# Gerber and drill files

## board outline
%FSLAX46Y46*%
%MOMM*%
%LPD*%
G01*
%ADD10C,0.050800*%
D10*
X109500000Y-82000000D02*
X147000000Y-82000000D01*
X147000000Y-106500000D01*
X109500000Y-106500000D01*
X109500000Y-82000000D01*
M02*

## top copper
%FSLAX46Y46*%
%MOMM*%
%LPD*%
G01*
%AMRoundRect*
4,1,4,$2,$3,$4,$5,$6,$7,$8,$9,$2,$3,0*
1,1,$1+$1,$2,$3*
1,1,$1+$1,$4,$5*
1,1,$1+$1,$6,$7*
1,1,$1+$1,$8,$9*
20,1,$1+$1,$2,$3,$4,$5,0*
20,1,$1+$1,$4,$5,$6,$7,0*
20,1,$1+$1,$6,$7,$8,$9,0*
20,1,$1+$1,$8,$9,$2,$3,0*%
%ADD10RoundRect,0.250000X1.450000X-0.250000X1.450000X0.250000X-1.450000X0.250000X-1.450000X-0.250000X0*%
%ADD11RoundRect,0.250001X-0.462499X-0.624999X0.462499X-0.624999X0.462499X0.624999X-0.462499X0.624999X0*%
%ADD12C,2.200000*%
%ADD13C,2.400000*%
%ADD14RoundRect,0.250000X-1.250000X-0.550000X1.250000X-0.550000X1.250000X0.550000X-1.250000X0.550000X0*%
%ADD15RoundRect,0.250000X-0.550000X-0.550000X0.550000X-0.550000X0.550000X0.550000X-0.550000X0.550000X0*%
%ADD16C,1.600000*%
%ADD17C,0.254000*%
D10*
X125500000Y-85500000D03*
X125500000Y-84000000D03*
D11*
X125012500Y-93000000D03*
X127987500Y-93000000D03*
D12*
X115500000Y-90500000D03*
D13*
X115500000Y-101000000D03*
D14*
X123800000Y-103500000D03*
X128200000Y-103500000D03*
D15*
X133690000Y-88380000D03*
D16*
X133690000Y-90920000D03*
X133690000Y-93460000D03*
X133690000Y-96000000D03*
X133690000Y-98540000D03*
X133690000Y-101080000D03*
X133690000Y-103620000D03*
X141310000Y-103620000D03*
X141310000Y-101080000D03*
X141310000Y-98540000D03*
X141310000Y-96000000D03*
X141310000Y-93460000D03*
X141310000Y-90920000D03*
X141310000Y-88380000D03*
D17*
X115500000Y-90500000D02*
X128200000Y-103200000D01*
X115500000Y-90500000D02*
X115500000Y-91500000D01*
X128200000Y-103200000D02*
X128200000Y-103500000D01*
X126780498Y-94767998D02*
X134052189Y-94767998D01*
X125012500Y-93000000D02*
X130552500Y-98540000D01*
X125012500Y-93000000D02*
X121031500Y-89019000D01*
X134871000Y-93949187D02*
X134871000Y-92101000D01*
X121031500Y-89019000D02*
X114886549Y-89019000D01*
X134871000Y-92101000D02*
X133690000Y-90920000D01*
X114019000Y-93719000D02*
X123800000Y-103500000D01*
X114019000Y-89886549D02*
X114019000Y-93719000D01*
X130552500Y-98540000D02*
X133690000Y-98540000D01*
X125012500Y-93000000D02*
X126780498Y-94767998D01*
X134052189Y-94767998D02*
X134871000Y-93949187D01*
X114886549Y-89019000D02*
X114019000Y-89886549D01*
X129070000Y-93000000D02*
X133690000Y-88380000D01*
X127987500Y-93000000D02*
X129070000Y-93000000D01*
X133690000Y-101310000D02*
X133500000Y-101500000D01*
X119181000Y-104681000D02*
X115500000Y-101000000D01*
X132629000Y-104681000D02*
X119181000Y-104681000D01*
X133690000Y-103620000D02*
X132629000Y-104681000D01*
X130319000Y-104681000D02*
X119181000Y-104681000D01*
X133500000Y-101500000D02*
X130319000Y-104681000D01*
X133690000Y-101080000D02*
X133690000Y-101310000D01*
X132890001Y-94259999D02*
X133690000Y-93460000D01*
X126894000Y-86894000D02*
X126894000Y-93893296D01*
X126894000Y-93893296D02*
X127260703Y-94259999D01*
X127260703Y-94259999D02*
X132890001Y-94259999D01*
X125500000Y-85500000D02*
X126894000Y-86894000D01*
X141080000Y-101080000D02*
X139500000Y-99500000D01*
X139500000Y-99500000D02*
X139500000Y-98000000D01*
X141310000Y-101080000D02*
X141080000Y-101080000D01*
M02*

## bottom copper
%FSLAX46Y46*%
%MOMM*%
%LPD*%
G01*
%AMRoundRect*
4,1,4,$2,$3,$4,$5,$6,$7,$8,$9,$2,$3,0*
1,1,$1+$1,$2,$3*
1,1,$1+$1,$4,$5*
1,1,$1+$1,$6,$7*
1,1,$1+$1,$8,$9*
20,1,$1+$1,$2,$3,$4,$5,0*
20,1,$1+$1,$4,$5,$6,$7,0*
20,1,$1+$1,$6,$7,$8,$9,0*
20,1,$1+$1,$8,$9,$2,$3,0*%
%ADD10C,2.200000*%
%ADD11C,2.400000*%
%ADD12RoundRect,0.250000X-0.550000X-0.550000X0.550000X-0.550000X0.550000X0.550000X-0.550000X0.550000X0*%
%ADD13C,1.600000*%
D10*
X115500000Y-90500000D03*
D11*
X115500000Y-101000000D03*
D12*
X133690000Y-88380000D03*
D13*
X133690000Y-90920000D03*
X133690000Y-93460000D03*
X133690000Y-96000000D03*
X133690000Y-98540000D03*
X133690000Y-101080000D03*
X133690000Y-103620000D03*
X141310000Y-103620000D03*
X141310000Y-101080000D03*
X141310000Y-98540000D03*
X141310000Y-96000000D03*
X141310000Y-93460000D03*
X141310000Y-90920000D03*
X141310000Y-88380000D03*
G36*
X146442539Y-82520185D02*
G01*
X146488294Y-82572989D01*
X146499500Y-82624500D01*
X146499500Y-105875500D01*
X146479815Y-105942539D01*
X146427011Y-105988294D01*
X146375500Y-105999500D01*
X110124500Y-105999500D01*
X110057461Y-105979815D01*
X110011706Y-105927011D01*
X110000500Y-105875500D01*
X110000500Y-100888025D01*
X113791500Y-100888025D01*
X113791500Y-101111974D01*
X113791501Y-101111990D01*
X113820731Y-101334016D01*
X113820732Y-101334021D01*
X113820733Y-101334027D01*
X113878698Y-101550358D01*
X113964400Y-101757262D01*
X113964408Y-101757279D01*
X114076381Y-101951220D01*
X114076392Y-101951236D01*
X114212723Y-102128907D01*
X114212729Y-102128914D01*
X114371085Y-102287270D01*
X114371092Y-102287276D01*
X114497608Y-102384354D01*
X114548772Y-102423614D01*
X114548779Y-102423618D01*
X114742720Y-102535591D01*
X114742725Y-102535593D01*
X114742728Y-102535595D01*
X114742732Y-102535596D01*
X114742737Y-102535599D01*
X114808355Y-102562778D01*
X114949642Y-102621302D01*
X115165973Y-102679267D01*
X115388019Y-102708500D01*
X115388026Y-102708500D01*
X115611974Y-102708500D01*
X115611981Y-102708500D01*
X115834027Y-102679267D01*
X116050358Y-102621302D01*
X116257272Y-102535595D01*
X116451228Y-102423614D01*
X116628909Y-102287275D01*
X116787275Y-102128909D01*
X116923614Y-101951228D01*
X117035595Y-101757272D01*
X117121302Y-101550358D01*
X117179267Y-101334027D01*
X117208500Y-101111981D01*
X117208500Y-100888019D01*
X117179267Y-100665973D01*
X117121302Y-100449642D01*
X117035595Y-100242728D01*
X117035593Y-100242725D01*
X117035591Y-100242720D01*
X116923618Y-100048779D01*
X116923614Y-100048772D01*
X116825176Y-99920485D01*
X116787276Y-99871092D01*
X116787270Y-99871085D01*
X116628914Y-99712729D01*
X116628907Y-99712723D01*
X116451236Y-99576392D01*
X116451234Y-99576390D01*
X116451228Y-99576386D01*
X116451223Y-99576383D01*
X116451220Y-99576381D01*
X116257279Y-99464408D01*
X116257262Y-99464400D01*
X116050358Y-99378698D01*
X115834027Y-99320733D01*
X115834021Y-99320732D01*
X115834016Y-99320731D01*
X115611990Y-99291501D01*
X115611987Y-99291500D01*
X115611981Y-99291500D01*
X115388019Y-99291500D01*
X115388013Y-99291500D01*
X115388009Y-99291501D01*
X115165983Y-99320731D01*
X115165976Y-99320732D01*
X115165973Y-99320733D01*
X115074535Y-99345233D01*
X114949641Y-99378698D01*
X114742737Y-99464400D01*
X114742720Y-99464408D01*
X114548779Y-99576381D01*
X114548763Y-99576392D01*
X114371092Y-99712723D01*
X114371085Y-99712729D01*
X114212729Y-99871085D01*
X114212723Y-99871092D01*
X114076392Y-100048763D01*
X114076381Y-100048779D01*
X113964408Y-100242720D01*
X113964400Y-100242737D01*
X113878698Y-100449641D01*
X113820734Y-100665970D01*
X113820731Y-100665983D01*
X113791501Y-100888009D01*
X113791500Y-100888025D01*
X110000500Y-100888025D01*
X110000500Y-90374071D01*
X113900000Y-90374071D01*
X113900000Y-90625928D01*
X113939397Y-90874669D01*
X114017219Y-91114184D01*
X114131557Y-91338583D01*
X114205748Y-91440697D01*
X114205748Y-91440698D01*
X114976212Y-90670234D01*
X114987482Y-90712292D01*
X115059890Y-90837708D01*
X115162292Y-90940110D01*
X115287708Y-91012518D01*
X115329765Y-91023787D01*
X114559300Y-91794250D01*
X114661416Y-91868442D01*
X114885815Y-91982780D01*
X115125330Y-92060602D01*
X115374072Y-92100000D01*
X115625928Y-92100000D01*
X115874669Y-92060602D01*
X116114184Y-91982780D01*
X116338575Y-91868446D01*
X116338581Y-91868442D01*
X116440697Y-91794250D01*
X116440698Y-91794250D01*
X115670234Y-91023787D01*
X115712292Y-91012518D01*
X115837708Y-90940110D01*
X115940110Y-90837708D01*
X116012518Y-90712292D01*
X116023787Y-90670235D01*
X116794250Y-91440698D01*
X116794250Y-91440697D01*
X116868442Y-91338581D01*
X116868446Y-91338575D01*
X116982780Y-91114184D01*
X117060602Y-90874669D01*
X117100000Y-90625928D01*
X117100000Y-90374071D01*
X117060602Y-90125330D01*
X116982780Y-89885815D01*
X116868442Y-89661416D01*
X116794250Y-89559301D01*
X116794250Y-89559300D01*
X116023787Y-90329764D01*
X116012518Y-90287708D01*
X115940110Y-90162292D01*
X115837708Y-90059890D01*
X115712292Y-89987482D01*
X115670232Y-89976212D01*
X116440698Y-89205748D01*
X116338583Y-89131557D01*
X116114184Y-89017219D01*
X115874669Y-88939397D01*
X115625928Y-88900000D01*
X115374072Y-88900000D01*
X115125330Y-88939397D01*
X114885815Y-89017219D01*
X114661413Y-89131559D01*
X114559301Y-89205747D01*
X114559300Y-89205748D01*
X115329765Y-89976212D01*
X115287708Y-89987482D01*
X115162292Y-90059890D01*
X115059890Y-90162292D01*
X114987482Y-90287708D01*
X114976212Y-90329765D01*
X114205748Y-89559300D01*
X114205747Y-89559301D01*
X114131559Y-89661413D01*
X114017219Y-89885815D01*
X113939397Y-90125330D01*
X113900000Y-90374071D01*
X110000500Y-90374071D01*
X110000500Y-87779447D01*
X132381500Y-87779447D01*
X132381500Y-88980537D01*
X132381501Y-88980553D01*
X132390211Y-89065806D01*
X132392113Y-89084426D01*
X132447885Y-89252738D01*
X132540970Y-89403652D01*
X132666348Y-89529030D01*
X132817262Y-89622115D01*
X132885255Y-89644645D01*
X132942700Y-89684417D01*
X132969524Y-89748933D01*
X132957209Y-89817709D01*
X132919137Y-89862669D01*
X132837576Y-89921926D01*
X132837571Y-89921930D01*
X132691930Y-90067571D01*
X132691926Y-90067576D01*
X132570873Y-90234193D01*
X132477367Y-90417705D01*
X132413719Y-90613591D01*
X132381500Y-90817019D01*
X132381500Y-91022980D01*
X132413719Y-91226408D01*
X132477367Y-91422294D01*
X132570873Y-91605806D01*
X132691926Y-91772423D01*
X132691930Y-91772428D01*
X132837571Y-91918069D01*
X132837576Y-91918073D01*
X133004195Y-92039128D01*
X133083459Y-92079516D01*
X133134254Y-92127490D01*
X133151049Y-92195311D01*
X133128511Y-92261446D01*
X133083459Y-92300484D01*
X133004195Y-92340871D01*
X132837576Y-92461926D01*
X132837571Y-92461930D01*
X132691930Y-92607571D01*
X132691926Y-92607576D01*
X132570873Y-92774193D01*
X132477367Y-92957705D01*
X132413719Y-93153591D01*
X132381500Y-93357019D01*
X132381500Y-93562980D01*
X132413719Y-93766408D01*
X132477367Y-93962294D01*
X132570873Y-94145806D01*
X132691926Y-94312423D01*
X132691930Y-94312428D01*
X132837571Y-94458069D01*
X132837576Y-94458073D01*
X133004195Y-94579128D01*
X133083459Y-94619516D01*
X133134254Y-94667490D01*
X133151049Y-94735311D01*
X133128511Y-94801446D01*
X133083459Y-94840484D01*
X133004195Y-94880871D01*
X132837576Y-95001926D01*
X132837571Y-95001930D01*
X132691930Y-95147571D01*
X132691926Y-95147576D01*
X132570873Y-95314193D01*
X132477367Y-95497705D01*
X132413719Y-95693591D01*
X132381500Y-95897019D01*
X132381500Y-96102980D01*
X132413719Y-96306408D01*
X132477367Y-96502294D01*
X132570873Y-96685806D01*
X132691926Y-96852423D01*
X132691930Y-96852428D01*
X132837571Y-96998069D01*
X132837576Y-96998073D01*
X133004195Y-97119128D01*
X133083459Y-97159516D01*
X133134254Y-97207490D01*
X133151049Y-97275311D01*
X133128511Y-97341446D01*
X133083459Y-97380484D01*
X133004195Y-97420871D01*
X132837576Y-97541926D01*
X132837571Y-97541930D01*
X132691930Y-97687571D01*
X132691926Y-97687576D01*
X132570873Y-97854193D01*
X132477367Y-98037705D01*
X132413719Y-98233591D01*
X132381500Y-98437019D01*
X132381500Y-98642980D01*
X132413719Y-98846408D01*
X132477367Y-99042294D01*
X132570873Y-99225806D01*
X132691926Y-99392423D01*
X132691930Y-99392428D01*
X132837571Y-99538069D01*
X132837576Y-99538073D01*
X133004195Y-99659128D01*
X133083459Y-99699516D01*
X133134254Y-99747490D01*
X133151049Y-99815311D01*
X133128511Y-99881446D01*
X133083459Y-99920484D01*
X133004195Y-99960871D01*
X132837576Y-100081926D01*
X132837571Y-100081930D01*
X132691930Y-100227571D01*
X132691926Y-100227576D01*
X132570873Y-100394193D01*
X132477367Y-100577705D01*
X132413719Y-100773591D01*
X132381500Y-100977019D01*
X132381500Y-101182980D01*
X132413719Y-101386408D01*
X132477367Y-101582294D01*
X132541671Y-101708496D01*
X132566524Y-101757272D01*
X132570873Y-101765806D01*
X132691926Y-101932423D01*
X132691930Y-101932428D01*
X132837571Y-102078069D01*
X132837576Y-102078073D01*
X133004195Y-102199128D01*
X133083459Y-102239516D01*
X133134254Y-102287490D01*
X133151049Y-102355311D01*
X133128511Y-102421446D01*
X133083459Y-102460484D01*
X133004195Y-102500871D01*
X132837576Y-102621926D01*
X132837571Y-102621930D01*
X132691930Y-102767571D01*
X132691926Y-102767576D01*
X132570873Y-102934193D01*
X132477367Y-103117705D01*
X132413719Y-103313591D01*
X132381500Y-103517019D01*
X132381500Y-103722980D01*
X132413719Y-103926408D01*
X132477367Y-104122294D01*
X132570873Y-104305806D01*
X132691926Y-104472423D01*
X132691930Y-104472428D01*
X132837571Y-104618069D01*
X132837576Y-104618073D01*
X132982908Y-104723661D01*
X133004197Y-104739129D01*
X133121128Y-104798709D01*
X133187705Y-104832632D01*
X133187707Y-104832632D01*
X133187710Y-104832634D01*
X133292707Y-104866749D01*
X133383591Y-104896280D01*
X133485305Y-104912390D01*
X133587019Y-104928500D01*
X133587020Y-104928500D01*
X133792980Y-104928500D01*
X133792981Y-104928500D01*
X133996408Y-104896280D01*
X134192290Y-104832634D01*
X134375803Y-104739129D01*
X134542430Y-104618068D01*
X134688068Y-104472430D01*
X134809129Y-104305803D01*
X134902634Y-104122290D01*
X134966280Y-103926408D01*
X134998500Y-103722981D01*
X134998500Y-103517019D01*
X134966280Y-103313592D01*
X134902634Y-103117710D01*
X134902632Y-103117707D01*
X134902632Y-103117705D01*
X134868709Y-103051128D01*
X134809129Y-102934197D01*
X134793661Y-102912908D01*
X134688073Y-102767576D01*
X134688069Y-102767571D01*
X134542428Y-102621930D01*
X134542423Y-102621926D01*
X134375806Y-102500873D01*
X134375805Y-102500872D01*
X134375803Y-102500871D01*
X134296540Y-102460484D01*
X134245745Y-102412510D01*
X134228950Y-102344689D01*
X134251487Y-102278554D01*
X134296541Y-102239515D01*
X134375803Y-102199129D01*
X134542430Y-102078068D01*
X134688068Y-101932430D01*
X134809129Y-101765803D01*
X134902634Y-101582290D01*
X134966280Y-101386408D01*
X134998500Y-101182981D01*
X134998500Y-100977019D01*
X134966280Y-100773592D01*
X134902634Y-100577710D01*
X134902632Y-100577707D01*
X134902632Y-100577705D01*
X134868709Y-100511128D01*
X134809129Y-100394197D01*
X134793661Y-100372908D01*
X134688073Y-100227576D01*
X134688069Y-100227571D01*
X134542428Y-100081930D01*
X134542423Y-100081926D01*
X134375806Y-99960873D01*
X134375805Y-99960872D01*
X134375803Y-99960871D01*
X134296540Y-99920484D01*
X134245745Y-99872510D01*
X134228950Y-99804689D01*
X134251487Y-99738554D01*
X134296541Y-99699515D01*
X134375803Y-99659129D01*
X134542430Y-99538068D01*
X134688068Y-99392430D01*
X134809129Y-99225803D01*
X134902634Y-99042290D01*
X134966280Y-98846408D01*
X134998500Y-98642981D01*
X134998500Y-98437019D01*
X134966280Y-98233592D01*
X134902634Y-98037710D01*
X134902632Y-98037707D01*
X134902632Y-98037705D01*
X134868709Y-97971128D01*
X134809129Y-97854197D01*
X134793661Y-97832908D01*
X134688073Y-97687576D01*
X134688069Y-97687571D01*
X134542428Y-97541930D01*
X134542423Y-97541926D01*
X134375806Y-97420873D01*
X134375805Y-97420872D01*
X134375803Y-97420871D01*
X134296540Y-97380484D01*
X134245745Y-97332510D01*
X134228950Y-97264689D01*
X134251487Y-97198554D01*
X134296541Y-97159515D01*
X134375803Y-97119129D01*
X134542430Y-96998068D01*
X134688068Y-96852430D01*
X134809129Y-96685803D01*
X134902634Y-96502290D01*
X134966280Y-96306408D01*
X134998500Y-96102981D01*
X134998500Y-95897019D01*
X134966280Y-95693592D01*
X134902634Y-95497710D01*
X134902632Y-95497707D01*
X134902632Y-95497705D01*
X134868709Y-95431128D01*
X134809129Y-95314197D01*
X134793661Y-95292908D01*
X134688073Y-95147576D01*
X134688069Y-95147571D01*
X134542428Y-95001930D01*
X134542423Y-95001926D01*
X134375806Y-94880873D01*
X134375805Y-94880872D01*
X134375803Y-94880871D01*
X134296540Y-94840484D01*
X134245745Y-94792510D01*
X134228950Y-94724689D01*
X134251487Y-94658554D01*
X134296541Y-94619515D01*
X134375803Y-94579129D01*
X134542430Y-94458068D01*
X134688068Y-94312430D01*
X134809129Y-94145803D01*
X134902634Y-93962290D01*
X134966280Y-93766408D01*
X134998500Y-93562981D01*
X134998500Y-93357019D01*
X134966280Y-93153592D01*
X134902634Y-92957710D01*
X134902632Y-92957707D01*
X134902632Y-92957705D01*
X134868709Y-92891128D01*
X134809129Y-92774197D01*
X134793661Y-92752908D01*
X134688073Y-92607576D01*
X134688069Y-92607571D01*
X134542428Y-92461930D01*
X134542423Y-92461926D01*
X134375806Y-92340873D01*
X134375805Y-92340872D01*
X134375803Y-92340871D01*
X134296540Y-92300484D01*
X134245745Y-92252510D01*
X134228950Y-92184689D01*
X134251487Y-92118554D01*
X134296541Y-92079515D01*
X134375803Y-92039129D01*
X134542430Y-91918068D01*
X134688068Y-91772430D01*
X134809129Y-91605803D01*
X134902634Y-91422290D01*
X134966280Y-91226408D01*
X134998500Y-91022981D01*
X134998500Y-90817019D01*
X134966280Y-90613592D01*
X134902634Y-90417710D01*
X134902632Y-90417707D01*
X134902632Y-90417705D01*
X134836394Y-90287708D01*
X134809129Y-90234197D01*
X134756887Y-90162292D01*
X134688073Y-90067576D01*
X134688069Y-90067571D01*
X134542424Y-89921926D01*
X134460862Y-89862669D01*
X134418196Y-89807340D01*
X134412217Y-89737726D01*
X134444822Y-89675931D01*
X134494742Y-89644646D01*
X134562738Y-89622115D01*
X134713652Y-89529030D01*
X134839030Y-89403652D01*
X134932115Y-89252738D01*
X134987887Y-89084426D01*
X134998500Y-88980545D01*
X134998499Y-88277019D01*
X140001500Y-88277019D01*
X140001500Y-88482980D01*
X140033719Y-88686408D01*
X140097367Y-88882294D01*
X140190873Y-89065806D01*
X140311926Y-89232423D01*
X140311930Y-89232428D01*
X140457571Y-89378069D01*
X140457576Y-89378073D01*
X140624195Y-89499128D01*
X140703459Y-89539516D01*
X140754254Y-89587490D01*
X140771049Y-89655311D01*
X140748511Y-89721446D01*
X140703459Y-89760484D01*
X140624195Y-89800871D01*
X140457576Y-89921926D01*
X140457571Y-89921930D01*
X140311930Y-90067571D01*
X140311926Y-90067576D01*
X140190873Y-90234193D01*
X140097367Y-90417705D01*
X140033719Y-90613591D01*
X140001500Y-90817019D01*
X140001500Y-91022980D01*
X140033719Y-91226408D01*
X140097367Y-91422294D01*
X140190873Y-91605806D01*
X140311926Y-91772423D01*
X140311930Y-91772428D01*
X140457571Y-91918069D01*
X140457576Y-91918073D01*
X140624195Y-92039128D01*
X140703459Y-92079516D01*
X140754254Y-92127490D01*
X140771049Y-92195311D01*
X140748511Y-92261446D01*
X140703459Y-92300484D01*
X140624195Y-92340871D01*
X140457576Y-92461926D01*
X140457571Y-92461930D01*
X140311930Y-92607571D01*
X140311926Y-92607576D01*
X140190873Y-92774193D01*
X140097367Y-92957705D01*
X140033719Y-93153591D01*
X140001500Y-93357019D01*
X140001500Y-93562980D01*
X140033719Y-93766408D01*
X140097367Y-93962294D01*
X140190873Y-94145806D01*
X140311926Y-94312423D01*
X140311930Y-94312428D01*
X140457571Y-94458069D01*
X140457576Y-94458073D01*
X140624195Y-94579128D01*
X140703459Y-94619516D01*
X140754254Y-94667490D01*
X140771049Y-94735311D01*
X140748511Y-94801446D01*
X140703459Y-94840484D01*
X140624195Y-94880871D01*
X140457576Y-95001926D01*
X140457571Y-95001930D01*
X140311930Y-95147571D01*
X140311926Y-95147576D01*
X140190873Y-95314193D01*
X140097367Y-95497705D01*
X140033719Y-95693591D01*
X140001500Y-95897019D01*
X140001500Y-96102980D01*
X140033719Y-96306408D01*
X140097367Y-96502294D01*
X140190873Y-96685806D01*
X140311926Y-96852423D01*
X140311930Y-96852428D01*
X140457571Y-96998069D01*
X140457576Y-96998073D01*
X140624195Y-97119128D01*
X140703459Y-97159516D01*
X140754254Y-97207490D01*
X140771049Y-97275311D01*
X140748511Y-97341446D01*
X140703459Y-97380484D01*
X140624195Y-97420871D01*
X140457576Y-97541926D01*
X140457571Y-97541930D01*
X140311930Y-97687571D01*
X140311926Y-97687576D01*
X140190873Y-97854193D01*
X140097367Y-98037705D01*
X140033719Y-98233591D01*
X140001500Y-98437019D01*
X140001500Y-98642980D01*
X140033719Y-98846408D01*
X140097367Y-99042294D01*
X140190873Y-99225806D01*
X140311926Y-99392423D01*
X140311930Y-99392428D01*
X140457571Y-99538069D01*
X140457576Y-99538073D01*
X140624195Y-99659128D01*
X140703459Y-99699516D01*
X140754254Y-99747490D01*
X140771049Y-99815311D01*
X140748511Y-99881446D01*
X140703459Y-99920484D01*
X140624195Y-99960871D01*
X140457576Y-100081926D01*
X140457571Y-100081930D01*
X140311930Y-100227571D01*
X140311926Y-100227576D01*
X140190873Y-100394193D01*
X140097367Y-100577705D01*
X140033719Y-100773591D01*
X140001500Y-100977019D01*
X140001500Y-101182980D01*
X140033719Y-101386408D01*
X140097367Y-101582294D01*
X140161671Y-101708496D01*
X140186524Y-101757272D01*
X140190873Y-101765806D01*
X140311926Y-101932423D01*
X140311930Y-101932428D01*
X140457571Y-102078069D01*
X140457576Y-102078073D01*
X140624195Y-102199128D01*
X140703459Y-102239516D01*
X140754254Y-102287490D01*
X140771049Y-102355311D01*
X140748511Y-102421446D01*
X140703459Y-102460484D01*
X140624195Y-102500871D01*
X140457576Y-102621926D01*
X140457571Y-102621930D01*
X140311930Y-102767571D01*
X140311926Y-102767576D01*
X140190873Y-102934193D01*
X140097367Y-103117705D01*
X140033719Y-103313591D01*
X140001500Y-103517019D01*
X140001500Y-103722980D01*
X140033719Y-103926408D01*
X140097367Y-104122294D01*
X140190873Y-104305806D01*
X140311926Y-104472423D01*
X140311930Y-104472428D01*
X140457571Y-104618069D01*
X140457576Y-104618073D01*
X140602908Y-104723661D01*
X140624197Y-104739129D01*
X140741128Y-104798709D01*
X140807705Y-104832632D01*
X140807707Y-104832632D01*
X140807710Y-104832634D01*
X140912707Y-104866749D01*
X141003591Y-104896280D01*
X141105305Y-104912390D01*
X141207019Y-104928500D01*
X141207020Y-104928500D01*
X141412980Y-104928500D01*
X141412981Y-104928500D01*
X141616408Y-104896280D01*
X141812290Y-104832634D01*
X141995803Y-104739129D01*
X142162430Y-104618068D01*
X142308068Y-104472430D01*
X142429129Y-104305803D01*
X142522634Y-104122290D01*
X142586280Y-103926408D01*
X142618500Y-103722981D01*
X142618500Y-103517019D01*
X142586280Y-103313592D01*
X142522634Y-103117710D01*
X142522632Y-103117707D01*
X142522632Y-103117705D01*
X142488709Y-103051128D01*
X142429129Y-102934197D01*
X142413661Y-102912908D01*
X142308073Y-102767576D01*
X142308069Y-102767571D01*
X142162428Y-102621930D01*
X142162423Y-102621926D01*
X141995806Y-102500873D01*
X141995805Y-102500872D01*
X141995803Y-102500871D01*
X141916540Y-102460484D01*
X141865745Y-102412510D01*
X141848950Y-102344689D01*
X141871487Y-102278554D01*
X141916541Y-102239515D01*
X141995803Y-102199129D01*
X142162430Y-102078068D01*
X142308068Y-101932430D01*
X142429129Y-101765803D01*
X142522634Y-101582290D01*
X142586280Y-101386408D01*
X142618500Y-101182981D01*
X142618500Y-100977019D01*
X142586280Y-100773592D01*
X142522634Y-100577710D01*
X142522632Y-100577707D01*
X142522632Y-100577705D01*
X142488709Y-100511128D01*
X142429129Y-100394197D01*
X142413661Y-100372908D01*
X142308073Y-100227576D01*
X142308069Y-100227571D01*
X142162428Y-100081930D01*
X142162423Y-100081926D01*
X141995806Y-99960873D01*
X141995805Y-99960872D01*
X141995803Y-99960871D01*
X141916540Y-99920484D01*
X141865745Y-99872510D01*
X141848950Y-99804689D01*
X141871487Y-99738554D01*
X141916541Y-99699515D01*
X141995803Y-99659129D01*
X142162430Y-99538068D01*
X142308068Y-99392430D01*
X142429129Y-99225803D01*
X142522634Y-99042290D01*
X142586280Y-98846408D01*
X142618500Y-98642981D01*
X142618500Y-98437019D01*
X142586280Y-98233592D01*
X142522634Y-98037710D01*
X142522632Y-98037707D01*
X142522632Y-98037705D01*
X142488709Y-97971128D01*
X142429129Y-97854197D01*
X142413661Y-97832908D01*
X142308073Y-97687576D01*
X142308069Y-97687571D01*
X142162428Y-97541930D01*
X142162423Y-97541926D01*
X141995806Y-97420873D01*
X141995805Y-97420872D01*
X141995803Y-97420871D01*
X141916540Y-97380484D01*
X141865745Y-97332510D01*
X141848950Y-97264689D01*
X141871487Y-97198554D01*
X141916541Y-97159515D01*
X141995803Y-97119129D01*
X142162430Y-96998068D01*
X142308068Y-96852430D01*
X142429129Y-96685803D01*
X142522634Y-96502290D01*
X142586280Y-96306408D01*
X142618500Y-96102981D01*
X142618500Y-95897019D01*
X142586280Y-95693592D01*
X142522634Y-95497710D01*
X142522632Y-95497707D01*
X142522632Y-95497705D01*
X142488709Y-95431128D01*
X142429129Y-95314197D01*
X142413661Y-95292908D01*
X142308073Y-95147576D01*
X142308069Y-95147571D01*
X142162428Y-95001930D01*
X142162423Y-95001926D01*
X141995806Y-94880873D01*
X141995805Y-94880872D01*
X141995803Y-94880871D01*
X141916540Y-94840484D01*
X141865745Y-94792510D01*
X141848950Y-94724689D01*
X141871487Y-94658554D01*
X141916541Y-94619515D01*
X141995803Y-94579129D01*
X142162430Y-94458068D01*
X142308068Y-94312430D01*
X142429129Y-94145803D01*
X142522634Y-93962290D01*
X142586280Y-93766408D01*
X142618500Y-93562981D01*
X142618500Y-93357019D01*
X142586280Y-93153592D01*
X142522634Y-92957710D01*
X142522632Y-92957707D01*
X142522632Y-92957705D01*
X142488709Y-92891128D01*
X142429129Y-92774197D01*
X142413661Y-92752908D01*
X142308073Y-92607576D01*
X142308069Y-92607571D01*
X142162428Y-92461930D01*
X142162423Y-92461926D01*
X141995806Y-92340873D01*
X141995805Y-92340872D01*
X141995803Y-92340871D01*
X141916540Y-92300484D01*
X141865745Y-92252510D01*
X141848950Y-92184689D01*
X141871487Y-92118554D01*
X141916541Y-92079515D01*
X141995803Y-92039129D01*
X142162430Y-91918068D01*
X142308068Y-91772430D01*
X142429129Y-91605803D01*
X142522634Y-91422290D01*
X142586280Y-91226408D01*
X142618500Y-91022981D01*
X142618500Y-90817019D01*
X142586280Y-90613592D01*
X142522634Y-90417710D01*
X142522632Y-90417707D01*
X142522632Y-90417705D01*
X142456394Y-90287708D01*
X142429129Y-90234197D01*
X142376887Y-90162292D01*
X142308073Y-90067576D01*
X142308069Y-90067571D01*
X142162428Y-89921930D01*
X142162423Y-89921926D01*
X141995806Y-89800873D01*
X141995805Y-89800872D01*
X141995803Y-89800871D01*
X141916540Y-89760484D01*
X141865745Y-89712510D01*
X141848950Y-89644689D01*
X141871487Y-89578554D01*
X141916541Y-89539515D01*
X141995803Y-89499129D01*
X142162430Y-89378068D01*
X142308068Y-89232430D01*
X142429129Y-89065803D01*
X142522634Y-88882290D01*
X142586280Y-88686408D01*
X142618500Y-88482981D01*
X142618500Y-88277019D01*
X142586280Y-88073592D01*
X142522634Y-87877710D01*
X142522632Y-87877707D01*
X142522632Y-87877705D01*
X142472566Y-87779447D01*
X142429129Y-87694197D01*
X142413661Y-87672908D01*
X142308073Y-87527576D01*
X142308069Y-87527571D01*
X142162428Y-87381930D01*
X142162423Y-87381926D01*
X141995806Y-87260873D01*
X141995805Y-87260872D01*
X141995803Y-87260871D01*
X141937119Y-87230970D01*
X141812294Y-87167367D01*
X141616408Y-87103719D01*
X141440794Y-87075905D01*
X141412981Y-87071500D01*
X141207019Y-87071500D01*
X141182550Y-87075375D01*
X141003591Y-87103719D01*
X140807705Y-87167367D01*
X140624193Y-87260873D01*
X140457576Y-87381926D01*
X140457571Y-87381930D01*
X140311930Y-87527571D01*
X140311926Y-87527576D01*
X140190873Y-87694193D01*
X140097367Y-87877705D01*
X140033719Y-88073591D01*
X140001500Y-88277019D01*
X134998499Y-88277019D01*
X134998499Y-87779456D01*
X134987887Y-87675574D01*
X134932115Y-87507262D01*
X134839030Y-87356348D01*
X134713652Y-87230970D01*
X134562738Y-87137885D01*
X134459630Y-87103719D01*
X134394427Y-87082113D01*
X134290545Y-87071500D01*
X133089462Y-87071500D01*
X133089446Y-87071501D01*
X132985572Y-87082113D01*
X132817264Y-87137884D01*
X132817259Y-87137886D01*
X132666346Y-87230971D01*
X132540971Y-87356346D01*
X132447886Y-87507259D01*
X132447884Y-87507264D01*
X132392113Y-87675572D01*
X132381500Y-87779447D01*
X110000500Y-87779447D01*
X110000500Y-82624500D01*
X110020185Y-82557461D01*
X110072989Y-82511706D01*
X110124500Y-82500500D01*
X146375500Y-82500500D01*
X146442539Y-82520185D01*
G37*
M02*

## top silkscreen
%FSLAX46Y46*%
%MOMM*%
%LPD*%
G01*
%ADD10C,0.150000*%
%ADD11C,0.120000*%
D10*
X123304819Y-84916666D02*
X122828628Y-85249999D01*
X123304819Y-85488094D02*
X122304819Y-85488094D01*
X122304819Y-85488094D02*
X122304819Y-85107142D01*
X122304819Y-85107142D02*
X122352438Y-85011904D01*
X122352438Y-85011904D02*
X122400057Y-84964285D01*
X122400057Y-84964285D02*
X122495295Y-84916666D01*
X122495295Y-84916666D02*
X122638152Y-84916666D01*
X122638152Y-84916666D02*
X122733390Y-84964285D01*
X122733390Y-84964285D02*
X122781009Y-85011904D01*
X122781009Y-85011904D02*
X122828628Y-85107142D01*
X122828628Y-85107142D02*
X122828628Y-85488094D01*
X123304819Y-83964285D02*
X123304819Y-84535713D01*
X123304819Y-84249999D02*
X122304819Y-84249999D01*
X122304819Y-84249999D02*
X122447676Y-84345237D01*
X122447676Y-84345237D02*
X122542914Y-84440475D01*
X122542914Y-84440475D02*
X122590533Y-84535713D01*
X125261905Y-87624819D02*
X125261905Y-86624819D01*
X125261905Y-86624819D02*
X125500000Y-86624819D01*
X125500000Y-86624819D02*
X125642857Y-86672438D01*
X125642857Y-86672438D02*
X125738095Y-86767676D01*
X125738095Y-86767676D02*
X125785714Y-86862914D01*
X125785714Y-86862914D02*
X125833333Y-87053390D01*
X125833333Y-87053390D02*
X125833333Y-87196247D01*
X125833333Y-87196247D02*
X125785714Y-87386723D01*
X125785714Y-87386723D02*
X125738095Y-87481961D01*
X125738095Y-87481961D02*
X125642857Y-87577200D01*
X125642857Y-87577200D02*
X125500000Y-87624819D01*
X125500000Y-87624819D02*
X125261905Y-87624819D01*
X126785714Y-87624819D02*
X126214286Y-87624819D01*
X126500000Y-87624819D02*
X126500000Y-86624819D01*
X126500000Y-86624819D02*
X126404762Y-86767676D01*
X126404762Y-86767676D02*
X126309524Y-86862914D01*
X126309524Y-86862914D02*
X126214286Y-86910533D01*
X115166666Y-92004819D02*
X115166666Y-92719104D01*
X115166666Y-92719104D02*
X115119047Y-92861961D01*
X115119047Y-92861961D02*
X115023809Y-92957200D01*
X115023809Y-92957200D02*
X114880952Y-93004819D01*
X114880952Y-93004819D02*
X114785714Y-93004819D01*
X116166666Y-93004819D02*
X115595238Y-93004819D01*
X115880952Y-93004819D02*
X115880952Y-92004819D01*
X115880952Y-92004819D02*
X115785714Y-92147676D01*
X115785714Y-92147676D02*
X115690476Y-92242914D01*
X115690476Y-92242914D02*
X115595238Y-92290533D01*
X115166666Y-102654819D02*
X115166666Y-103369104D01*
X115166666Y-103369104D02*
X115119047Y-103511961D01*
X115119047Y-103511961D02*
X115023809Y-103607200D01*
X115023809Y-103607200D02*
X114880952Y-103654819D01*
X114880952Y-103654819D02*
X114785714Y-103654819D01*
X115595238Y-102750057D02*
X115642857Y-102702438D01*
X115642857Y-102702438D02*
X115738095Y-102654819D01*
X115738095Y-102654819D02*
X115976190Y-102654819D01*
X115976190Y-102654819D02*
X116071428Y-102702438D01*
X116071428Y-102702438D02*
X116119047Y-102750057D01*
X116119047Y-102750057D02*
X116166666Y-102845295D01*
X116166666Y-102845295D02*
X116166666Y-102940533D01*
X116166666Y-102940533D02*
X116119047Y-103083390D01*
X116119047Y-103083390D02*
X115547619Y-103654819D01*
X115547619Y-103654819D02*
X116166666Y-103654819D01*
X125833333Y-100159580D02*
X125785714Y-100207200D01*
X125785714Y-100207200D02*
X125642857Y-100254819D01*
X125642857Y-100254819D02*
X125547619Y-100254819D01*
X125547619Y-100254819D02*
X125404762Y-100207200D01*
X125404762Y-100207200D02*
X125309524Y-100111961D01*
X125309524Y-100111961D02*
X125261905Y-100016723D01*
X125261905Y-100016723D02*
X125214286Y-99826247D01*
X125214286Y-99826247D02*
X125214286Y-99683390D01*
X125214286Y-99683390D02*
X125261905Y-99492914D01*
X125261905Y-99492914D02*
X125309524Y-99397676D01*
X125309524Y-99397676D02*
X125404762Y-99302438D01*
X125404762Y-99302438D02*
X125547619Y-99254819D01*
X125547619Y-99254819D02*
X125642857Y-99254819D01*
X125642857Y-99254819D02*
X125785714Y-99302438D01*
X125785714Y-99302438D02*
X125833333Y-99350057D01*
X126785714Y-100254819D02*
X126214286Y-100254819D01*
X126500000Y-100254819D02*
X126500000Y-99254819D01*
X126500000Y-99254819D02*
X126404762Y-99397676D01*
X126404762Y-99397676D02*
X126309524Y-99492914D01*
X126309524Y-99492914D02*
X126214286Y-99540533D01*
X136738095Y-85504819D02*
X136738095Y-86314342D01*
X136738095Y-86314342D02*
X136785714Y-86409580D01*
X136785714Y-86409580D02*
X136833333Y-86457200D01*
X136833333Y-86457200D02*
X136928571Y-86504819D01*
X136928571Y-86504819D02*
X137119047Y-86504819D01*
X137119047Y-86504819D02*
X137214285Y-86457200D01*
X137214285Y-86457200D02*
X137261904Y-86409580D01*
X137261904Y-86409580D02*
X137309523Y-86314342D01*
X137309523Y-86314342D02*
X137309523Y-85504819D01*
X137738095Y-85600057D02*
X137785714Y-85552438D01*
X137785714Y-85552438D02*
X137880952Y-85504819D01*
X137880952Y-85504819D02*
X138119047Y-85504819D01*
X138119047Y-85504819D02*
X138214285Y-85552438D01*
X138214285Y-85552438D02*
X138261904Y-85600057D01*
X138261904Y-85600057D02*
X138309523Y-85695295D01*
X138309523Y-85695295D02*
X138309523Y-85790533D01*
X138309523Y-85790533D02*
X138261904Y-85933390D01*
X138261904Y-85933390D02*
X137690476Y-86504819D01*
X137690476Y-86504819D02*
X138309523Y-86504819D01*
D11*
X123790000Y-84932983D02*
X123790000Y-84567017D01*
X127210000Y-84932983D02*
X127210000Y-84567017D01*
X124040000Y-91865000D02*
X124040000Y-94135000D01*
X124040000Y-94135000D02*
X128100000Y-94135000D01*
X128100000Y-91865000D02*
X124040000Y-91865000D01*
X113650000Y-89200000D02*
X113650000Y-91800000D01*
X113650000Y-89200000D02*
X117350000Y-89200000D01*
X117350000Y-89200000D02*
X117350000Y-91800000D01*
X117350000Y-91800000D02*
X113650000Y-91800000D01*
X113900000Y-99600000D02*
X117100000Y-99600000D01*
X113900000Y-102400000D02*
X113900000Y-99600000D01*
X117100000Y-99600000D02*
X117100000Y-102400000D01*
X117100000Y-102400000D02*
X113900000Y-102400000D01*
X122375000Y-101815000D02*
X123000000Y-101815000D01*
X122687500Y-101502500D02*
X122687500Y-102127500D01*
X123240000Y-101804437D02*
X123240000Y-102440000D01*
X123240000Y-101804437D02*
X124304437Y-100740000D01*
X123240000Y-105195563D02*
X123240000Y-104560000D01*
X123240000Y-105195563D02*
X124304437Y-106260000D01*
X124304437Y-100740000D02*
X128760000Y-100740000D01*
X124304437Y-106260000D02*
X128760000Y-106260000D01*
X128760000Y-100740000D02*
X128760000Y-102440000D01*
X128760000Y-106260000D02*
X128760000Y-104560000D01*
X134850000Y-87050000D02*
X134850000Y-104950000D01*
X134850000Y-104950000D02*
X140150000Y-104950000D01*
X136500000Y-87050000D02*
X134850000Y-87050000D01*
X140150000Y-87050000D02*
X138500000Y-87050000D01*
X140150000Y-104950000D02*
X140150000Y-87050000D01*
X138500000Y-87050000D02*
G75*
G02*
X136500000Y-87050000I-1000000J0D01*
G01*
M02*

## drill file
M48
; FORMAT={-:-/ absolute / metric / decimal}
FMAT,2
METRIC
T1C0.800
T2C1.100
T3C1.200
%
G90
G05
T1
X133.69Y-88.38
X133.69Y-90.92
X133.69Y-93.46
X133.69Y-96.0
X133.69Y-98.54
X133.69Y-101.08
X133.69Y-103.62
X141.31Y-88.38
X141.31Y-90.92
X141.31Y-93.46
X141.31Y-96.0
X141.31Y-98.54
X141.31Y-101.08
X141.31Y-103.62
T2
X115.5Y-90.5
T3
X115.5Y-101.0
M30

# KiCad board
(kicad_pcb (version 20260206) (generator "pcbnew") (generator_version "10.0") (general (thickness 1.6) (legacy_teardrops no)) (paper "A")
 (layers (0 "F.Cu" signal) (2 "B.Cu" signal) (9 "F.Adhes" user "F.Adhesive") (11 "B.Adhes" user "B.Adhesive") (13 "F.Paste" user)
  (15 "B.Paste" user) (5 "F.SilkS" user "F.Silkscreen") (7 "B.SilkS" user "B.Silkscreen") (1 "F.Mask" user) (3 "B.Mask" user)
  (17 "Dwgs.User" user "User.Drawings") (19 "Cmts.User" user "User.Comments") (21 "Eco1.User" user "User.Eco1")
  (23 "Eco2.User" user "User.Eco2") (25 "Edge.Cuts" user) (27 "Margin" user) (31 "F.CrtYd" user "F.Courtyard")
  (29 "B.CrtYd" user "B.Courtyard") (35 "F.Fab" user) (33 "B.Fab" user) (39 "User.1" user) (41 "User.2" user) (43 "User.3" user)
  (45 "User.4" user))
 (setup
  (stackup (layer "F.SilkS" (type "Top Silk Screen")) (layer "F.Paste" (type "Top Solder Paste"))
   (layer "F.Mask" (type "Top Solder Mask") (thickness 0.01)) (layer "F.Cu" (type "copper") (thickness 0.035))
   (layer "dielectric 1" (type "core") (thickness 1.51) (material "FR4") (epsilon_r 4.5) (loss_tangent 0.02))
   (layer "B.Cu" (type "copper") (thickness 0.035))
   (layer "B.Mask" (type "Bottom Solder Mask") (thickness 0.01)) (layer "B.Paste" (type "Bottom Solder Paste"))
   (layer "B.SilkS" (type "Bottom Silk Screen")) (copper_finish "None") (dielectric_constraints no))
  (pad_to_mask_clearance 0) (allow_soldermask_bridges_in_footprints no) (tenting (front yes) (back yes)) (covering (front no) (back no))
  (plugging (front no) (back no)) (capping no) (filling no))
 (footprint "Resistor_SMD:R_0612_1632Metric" (layer "F.Cu") (at 125.5 84.75 90)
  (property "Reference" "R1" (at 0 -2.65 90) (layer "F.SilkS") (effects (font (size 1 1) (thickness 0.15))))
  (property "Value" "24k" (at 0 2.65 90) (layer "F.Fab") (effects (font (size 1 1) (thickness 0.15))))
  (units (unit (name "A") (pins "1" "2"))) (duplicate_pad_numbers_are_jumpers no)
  (fp_line (start -0.182983 -1.71) (end 0.182983 -1.71) (stroke (width 0.12) (type solid)) (layer "F.SilkS"))
  (fp_line (start -0.182983 1.71) (end 0.182983 1.71) (stroke (width 0.12) (type solid)) (layer "F.SilkS"))
  (pad "1" smd roundrect (at -0.75 0 90) (size 1 3.4) (layers "F.Cu" "F.Mask" "F.Paste") (roundrect_rratio 0.25) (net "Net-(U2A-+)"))
  (pad "2" smd roundrect (at 0.75 0 90) (size 1 3.4) (layers "F.Cu" "F.Mask" "F.Paste") (roundrect_rratio 0.25) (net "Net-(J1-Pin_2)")))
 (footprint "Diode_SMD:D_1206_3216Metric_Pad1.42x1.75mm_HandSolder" (layer "F.Cu") (at 126.5 93)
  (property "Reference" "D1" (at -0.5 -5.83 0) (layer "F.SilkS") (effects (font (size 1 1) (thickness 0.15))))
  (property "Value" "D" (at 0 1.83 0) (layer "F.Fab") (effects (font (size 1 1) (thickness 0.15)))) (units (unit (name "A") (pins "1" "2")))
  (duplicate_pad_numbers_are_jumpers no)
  (fp_line (start -2.46 -1.135) (end -2.46 1.135) (stroke (width 0.12) (type solid)) (layer "F.SilkS"))
  (fp_line (start -2.46 1.135) (end 1.6 1.135) (stroke (width 0.12) (type solid)) (layer "F.SilkS"))
  (fp_line (start 1.6 -1.135) (end -2.46 -1.135) (stroke (width 0.12) (type solid)) (layer "F.SilkS"))
  (pad "1" smd roundrect (at -1.4875 0) (size 1.425 1.75) (layers "F.Cu" "F.Mask" "F.Paste") (roundrect_rratio 0.175439) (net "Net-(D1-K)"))
  (pad "2" smd roundrect (at 1.4875 0) (size 1.425 1.75) (layers "F.Cu" "F.Mask" "F.Paste") (roundrect_rratio 0.175439) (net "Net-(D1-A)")))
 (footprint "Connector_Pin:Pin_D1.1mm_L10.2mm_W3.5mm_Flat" (layer "F.Cu") (at 115.5 90.5)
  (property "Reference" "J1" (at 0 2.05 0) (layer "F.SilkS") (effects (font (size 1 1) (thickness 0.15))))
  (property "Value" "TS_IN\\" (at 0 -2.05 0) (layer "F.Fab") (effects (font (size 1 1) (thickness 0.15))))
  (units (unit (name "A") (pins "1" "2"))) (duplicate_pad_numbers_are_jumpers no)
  (fp_line (start -1.85 -1.3) (end -1.85 1.3) (stroke (width 0.12) (type solid)) (layer "F.SilkS"))
  (fp_line (start -1.85 -1.3) (end 1.85 -1.3) (stroke (width 0.12) (type solid)) (layer "F.SilkS"))
  (fp_line (start 1.85 -1.3) (end 1.85 1.3) (stroke (width 0.12) (type solid)) (layer "F.SilkS"))
  (fp_line (start 1.85 1.3) (end -1.85 1.3) (stroke (width 0.12) (type solid)) (layer "F.SilkS"))
  (pad "1" thru_hole circle (at 0 0) (size 2.2 2.2) (drill 1.1) (layers "*.Cu" "*.Mask") (remove_unused_layers no) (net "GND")))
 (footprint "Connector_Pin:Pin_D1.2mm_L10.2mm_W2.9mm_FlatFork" (layer "F.Cu") (at 115.5 101)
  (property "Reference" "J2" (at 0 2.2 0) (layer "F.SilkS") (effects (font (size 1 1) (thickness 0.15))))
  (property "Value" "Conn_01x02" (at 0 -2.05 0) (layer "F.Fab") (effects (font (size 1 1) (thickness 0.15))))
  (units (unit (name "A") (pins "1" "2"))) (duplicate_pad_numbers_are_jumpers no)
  (fp_line (start -1.6 -1.4) (end 1.6 -1.4) (stroke (width 0.12) (type solid)) (layer "F.SilkS"))
  (fp_line (start -1.6 1.4) (end -1.6 -1.4) (stroke (width 0.12) (type solid)) (layer "F.SilkS"))
  (fp_line (start 1.6 -1.4) (end 1.6 1.4) (stroke (width 0.12) (type solid)) (layer "F.SilkS"))
  (fp_line (start 1.6 1.4) (end -1.6 1.4) (stroke (width 0.12) (type solid)) (layer "F.SilkS"))
  (pad "1" thru_hole circle (at 0 0) (size 2.4 2.4) (drill 1.2) (layers "*.Cu" "*.Mask") (remove_unused_layers no) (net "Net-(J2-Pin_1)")))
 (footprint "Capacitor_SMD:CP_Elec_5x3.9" (layer "F.Cu") (at 126 103.5)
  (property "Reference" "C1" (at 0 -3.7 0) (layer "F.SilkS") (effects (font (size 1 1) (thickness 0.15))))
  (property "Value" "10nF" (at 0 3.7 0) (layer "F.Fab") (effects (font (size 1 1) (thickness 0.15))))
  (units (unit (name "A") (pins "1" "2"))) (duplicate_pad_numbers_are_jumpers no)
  (fp_line (start -3.625 -1.685) (end -3 -1.685) (stroke (width 0.12) (type solid)) (layer "F.SilkS"))
  (fp_line (start -3.3125 -1.9975) (end -3.3125 -1.3725) (stroke (width 0.12) (type solid)) (layer "F.SilkS"))
  (fp_line (start -2.76 -1.695563) (end -2.76 -1.06) (stroke (width 0.12) (type solid)) (layer "F.SilkS"))
  (fp_line (start -2.76 -1.695563) (end -1.695563 -2.76) (stroke (width 0.12) (type solid)) (layer "F.SilkS"))
  (fp_line (start -2.76 1.695563) (end -2.76 1.06) (stroke (width 0.12) (type solid)) (layer "F.SilkS"))
  (fp_line (start -2.76 1.695563) (end -1.695563 2.76) (stroke (width 0.12) (type solid)) (layer "F.SilkS"))
  (fp_line (start -1.695563 -2.76) (end 2.76 -2.76) (stroke (width 0.12) (type solid)) (layer "F.SilkS"))
  (fp_line (start -1.695563 2.76) (end 2.76 2.76) (stroke (width 0.12) (type solid)) (layer "F.SilkS"))
  (fp_line (start 2.76 -2.76) (end 2.76 -1.06) (stroke (width 0.12) (type solid)) (layer "F.SilkS"))
  (fp_line (start 2.76 2.76) (end 2.76 1.06) (stroke (width 0.12) (type solid)) (layer "F.SilkS"))
  (pad "1" smd roundrect (at -2.2 0) (size 3 1.6) (layers "F.Cu" "F.Mask" "F.Paste") (roundrect_rratio 0.15625) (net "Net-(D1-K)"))
  (pad "2" smd roundrect (at 2.2 0) (size 3 1.6) (layers "F.Cu" "F.Mask" "F.Paste") (roundrect_rratio 0.15625) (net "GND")))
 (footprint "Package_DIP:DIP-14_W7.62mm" (layer "F.Cu") (at 133.69 88.38)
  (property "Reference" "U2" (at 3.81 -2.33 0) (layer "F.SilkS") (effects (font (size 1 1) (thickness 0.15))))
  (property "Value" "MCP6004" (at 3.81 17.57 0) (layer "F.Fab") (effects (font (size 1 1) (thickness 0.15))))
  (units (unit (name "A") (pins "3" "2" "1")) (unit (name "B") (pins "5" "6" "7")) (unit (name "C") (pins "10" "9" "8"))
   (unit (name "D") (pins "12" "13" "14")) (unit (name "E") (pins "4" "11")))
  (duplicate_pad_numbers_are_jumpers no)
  (fp_line (start 1.16 -1.33) (end 1.16 16.57) (stroke (width 0.12) (type solid)) (layer "F.SilkS"))
  (fp_line (start 1.16 16.57) (end 6.46 16.57) (stroke (width 0.12) (type solid)) (layer "F.SilkS"))
  (fp_line (start 2.81 -1.33) (end 1.16 -1.33) (stroke (width 0.12) (type solid)) (layer "F.SilkS"))
  (fp_line (start 6.46 -1.33) (end 4.81 -1.33) (stroke (width 0.12) (type solid)) (layer "F.SilkS"))
  (fp_line (start 6.46 16.57) (end 6.46 -1.33) (stroke (width 0.12) (type solid)) (layer "F.SilkS"))
  (fp_arc (start 4.81 -1.33) (mid 3.81 -0.33) (end 2.81 -1.33) (stroke (width 0.12) (type solid)) (layer "F.SilkS"))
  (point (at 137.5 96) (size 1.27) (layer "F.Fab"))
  (pad "1" thru_hole roundrect (at 0 0) (size 1.6 1.6) (drill 0.8) (layers "*.Cu" "*.Mask") (remove_unused_layers no)
   (roundrect_rratio 0.15625) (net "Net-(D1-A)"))
  (pad "2" thru_hole circle (at 0 2.54) (size 1.6 1.6) (drill 0.8) (layers "*.Cu" "*.Mask") (remove_unused_layers no) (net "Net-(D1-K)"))
  (pad "3" thru_hole circle (at 0 5.08) (size 1.6 1.6) (drill 0.8) (layers "*.Cu" "*.Mask") (remove_unused_layers no) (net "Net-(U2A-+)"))
  (pad "4" thru_hole circle (at 0 7.62) (size 1.6 1.6) (drill 0.8) (layers "*.Cu" "*.Mask") (remove_unused_layers no))
  (pad "5" thru_hole circle (at 0 10.16) (size 1.6 1.6) (drill 0.8) (layers "*.Cu" "*.Mask") (remove_unused_layers no) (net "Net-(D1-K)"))
  (pad "6" thru_hole circle (at 0 12.7) (size 1.6 1.6) (drill 0.8) (layers "*.Cu" "*.Mask") (remove_unused_layers no) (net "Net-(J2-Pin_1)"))
  (pad "7" thru_hole circle (at 0 15.24) (size 1.6 1.6) (drill 0.8) (layers "*.Cu" "*.Mask") (remove_unused_layers no)
   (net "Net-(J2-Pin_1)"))
  (pad "8" thru_hole circle (at 7.62 15.24) (size 1.6 1.6) (drill 0.8) (layers "*.Cu" "*.Mask") (remove_unused_layers no)
   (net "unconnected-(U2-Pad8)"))
  (pad "9" thru_hole circle (at 7.62 12.7) (size 1.6 1.6) (drill 0.8) (layers "*.Cu" "*.Mask") (remove_unused_layers no)
   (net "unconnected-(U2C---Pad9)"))
  (pad "10" thru_hole circle (at 7.62 10.16) (size 1.6 1.6) (drill 0.8) (layers "*.Cu" "*.Mask") (remove_unused_layers no)
   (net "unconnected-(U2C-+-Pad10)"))
  (pad "11" thru_hole circle (at 7.62 7.62) (size 1.6 1.6) (drill 0.8) (layers "*.Cu" "*.Mask") (remove_unused_layers no))
  (pad "12" thru_hole circle (at 7.62 5.08) (size 1.6 1.6) (drill 0.8) (layers "*.Cu" "*.Mask") (remove_unused_layers no)
   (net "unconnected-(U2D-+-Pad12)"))
  (pad "13" thru_hole circle (at 7.62 2.54) (size 1.6 1.6) (drill 0.8) (layers "*.Cu" "*.Mask") (remove_unused_layers no)
   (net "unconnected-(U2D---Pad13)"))
  (pad "14" thru_hole circle (at 7.62 0) (size 1.6 1.6) (drill 0.8) (layers "*.Cu" "*.Mask") (remove_unused_layers no)
   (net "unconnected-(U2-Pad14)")))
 (gr_rect (start 109.5 82) (end 147 106.5) (stroke (width 0.0508) (type default)) (fill no) (layer "Edge.Cuts"))
 (segment (start 115.5 90.5) (end 128.2 103.2) (width 0.254) (layer "F.Cu") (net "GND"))
 (segment (start 115.5 90.5) (end 115.5 91.5) (width 0.254) (layer "F.Cu") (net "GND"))
 (segment (start 128.2 103.2) (end 128.2 103.5) (width 0.254) (layer "F.Cu") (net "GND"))
 (segment (start 126.780498 94.767998) (end 134.052189 94.767998) (width 0.254) (layer "F.Cu") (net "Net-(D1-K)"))
 (segment (start 125.0125 93) (end 130.5525 98.54) (width 0.254) (layer "F.Cu") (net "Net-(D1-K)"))
 (segment (start 125.0125 93) (end 121.0315 89.019) (width 0.254) (layer "F.Cu") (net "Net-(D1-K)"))
 (segment (start 134.871 93.949187) (end 134.871 92.101) (width 0.254) (layer "F.Cu") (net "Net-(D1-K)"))
 (segment (start 121.0315 89.019) (end 114.886549 89.019) (width 0.254) (layer "F.Cu") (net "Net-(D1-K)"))
 (segment (start 134.871 92.101) (end 133.69 90.92) (width 0.254) (layer "F.Cu") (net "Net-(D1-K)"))
 (segment (start 114.019 93.719) (end 123.8 103.5) (width 0.254) (layer "F.Cu") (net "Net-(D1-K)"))
 (segment (start 114.019 89.886549) (end 114.019 93.719) (width 0.254) (layer "F.Cu") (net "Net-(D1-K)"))
 (segment (start 130.5525 98.54) (end 133.69 98.54) (width 0.254) (layer "F.Cu") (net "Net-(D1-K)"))
 (segment (start 125.0125 93) (end 126.780498 94.767998) (width 0.254) (layer "F.Cu") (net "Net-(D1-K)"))
 (segment (start 134.052189 94.767998) (end 134.871 93.949187) (width 0.254) (layer "F.Cu") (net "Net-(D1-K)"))
 (segment (start 114.886549 89.019) (end 114.019 89.886549) (width 0.254) (layer "F.Cu") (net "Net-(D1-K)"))
 (segment (start 129.07 93) (end 133.69 88.38) (width 0.254) (layer "F.Cu") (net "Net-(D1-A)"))
 (segment (start 127.9875 93) (end 129.07 93) (width 0.254) (layer "F.Cu") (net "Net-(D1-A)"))
 (segment (start 133.69 101.31) (end 133.5 101.5) (width 0.254) (layer "F.Cu") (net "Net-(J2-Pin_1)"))
 (segment (start 119.181 104.681) (end 115.5 101) (width 0.254) (layer "F.Cu") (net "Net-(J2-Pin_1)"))
 (segment (start 132.629 104.681) (end 119.181 104.681) (width 0.254) (layer "F.Cu") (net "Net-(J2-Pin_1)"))
 (segment (start 133.69 103.62) (end 132.629 104.681) (width 0.254) (layer "F.Cu") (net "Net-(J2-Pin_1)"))
 (segment (start 130.319 104.681) (end 119.181 104.681) (width 0.254) (layer "F.Cu") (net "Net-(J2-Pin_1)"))
 (segment (start 133.5 101.5) (end 130.319 104.681) (width 0.254) (layer "F.Cu") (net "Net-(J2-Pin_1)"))
 (segment (start 133.69 101.08) (end 133.69 101.31) (width 0.254) (layer "F.Cu") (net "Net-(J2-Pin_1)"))
 (segment (start 132.890001 94.259999) (end 133.69 93.46) (width 0.254) (layer "F.Cu") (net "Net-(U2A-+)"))
 (segment (start 126.894 86.894) (end 126.894 93.893296) (width 0.254) (layer "F.Cu") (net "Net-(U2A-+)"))
 (segment (start 126.894 93.893296) (end 127.260703 94.259999) (width 0.254) (layer "F.Cu") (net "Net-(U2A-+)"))
 (segment (start 127.260703 94.259999) (end 132.890001 94.259999) (width 0.254) (layer "F.Cu") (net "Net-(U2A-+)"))
 (segment (start 125.5 85.5) (end 126.894 86.894) (width 0.254) (layer "F.Cu") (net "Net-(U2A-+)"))
 (segment (start 141.08 101.08) (end 139.5 99.5) (width 0.254) (layer "F.Cu") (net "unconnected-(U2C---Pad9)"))
 (segment (start 139.5 99.5) (end 139.5 98) (width 0.254) (layer "F.Cu") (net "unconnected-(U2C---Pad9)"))
 (segment (start 141.31 101.08) (end 141.08 101.08) (width 0.254) (layer "F.Cu") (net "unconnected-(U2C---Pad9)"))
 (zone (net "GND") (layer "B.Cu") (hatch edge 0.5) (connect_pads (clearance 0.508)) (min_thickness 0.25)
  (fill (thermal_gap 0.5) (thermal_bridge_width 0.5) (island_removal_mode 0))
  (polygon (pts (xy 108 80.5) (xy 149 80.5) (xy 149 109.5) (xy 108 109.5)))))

